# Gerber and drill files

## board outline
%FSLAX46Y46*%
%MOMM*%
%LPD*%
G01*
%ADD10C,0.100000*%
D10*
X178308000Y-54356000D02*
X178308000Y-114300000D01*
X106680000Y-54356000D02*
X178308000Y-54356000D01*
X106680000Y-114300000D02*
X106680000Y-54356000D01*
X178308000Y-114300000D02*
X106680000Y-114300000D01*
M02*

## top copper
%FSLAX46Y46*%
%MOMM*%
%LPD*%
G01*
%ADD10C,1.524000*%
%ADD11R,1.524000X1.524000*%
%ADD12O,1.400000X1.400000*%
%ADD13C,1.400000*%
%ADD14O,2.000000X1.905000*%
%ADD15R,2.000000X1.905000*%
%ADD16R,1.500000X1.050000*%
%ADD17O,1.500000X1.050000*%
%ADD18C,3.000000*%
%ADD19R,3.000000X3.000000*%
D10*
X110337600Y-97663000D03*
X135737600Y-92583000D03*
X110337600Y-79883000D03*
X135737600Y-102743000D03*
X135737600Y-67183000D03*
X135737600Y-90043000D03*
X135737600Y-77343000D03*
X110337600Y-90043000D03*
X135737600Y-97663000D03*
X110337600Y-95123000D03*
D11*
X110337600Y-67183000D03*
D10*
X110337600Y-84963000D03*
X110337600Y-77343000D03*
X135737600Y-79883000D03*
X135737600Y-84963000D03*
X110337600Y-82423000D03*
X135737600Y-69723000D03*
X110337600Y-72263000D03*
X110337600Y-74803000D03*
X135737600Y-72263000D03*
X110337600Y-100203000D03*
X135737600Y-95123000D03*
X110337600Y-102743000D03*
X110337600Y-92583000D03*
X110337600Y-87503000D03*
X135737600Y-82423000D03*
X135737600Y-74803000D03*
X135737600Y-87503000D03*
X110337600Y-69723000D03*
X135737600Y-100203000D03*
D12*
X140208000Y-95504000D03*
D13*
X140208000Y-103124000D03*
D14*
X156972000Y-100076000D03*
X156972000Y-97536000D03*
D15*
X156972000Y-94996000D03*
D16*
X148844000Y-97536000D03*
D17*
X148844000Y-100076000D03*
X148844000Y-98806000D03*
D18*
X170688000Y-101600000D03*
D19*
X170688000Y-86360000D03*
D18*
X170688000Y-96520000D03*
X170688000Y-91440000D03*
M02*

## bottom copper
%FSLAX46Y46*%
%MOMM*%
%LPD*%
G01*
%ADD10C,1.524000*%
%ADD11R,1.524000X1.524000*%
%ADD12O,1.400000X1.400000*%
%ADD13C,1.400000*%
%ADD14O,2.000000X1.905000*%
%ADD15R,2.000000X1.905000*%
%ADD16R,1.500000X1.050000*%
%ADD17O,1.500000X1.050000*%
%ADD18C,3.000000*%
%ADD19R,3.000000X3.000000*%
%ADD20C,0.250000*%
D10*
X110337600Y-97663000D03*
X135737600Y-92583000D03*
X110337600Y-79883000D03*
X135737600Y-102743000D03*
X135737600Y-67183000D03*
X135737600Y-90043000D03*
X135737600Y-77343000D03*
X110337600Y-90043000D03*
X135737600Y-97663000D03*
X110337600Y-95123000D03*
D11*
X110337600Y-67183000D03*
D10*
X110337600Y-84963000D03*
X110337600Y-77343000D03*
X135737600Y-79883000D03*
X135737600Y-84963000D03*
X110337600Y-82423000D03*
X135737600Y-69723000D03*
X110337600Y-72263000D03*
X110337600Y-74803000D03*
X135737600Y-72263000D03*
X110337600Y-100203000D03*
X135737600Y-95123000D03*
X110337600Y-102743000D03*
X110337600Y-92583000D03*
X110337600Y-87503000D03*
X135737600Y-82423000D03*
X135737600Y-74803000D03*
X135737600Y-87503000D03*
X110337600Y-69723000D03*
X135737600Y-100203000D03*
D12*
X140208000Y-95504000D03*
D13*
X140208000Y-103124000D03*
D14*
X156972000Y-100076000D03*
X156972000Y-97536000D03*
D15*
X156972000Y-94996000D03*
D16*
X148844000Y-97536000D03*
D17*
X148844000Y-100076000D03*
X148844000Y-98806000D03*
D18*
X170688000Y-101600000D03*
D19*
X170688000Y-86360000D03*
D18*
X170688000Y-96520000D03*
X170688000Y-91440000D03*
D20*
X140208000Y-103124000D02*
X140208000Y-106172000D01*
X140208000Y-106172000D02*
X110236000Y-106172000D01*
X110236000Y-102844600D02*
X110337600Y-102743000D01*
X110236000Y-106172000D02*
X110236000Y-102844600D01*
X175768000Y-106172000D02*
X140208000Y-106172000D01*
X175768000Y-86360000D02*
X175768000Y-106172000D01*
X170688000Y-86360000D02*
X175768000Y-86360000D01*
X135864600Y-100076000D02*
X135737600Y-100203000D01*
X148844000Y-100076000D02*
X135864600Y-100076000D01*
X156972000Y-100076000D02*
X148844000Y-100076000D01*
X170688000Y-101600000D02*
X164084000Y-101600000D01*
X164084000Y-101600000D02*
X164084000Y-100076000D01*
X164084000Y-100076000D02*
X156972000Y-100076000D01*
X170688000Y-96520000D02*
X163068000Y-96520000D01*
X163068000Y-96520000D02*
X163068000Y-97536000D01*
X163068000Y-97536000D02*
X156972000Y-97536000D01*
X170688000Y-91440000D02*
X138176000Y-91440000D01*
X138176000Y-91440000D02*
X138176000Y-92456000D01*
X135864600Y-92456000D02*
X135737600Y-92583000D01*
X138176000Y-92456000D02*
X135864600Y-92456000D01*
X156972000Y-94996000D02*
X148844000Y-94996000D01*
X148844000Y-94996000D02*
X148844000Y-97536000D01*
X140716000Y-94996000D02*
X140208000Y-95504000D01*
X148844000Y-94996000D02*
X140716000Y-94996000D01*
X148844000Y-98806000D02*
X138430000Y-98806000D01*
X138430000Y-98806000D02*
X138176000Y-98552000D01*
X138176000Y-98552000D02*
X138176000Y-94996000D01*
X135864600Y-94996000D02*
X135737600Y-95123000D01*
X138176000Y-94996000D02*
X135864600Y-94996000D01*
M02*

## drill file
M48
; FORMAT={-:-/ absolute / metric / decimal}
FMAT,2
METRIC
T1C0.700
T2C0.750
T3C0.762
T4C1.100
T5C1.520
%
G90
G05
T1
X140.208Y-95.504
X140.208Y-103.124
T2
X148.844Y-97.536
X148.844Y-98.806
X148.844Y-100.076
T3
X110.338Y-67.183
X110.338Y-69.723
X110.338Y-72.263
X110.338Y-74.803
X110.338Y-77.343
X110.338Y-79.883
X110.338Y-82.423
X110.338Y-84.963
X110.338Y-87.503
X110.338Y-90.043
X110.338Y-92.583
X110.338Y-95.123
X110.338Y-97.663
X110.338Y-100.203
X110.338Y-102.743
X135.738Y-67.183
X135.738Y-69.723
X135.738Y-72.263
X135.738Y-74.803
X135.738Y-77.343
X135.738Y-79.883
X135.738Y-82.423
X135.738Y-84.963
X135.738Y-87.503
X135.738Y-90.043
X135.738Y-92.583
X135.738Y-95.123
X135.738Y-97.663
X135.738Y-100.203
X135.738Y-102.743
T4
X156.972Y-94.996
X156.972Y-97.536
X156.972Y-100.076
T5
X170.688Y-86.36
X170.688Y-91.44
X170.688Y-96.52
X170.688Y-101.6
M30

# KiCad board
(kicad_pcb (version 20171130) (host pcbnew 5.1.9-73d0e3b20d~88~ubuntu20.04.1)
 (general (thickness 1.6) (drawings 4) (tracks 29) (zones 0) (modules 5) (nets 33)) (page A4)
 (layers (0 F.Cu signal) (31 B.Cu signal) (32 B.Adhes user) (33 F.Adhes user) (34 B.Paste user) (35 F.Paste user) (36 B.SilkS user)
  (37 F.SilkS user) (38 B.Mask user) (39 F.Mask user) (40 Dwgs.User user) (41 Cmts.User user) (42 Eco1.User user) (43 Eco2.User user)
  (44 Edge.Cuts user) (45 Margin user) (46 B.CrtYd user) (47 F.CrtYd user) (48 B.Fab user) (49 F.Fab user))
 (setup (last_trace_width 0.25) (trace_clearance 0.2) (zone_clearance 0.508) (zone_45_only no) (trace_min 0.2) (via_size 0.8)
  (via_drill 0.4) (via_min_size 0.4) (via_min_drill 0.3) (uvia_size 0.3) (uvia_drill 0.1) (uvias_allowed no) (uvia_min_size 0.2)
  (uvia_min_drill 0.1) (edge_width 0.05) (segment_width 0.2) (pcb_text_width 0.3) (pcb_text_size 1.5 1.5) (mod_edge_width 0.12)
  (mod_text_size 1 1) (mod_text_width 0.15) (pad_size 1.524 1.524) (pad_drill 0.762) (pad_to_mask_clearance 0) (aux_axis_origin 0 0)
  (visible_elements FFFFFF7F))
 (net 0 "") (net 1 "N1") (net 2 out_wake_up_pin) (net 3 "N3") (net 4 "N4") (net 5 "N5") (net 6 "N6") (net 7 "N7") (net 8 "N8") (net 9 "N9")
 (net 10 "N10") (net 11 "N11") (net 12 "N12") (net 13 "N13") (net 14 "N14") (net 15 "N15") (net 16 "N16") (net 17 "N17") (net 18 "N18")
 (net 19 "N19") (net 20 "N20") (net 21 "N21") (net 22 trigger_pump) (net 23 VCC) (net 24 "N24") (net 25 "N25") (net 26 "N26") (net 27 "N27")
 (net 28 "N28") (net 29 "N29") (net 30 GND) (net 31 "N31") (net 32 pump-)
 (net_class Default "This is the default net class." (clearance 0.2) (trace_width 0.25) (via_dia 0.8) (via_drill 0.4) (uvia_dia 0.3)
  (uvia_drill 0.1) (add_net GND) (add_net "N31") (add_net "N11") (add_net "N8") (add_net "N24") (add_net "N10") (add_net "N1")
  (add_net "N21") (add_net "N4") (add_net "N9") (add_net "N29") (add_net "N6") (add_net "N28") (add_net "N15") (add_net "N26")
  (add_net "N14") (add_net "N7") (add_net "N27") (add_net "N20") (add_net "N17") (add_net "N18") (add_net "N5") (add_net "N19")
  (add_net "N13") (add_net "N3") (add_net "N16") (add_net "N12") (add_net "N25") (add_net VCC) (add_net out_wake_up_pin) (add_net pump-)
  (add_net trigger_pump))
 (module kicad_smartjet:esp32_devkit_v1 (layer F.Cu) (at 121.92 58.42)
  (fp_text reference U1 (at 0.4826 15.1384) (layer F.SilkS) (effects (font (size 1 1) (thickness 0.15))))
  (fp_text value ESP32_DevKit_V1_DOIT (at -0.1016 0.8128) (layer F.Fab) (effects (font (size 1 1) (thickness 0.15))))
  (pad 13 thru_hole circle (at -11.5824 39.243) (size 1.524 1.524) (drill 0.762) (layers *.Cu *.Mask) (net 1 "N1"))
  (pad 20 thru_hole circle (at 13.8176 34.163) (size 1.524 1.524) (drill 0.762) (layers *.Cu *.Mask) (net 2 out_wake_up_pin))
  (pad 6 thru_hole circle (at -11.5824 21.463) (size 1.524 1.524) (drill 0.762) (layers *.Cu *.Mask) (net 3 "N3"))
  (pad 16 thru_hole circle (at 13.8176 44.323) (size 1.524 1.524) (drill 0.762) (layers *.Cu *.Mask) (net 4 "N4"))
  (pad 30 thru_hole circle (at 13.8176 8.763) (size 1.524 1.524) (drill 0.762) (layers *.Cu *.Mask) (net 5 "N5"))
  (pad 21 thru_hole circle (at 13.8176 31.623) (size 1.524 1.524) (drill 0.762) (layers *.Cu *.Mask) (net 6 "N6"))
  (pad 26 thru_hole circle (at 13.8176 18.923) (size 1.524 1.524) (drill 0.762) (layers *.Cu *.Mask) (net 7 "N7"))
  (pad 10 thru_hole circle (at -11.5824 31.623) (size 1.524 1.524) (drill 0.762) (layers *.Cu *.Mask) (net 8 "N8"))
  (pad 18 thru_hole circle (at 13.8176 39.243) (size 1.524 1.524) (drill 0.762) (layers *.Cu *.Mask) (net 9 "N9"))
  (pad 12 thru_hole circle (at -11.5824 36.703) (size 1.524 1.524) (drill 0.762) (layers *.Cu *.Mask) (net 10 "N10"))
  (pad 1 thru_hole rect (at -11.5824 8.763) (size 1.524 1.524) (drill 0.762) (layers *.Cu *.Mask) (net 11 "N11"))
  (pad 8 thru_hole circle (at -11.5824 26.543) (size 1.524 1.524) (drill 0.762) (layers *.Cu *.Mask) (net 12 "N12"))
  (pad 5 thru_hole circle (at -11.5824 18.923) (size 1.524 1.524) (drill 0.762) (layers *.Cu *.Mask) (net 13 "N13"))
  (pad 25 thru_hole circle (at 13.8176 21.463) (size 1.524 1.524) (drill 0.762) (layers *.Cu *.Mask) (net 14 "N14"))
  (pad 23 thru_hole circle (at 13.8176 26.543) (size 1.524 1.524) (drill 0.762) (layers *.Cu *.Mask) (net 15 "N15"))
  (pad 7 thru_hole circle (at -11.5824 24.003) (size 1.524 1.524) (drill 0.762) (layers *.Cu *.Mask) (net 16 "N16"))
  (pad 29 thru_hole circle (at 13.8176 11.303) (size 1.524 1.524) (drill 0.762) (layers *.Cu *.Mask) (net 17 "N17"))
  (pad 3 thru_hole circle (at -11.5824 13.843) (size 1.524 1.524) (drill 0.762) (layers *.Cu *.Mask) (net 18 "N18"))
  (pad 4 thru_hole circle (at -11.5824 16.383) (size 1.524 1.524) (drill 0.762) (layers *.Cu *.Mask) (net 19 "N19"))
  (pad 28 thru_hole circle (at 13.8176 13.843) (size 1.524 1.524) (drill 0.762) (layers *.Cu *.Mask) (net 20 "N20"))
  (pad 14 thru_hole circle (at -11.5824 41.783) (size 1.524 1.524) (drill 0.762) (layers *.Cu *.Mask) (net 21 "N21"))
  (pad 19 thru_hole circle (at 13.8176 36.703) (size 1.524 1.524) (drill 0.762) (layers *.Cu *.Mask) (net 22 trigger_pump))
  (pad 15 thru_hole circle (at -11.5824 44.323) (size 1.524 1.524) (drill 0.762) (layers *.Cu *.Mask) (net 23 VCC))
  (pad 11 thru_hole circle (at -11.5824 34.163) (size 1.524 1.524) (drill 0.762) (layers *.Cu *.Mask) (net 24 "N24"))
  (pad 9 thru_hole circle (at -11.5824 29.083) (size 1.524 1.524) (drill 0.762) (layers *.Cu *.Mask) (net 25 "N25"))
  (pad 24 thru_hole circle (at 13.8176 24.003) (size 1.524 1.524) (drill 0.762) (layers *.Cu *.Mask) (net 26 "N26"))
  (pad 27 thru_hole circle (at 13.8176 16.383) (size 1.524 1.524) (drill 0.762) (layers *.Cu *.Mask) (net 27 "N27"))
  (pad 22 thru_hole circle (at 13.8176 29.083) (size 1.524 1.524) (drill 0.762) (layers *.Cu *.Mask) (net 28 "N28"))
  (pad 2 thru_hole circle (at -11.5824 11.303) (size 1.524 1.524) (drill 0.762) (layers *.Cu *.Mask) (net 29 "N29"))
  (pad 17 thru_hole circle (at 13.8176 41.783) (size 1.524 1.524) (drill 0.762) (layers *.Cu *.Mask) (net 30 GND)))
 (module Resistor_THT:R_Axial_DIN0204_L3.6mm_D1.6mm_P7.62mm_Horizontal (layer F.Cu) (at 140.208 103.124 90)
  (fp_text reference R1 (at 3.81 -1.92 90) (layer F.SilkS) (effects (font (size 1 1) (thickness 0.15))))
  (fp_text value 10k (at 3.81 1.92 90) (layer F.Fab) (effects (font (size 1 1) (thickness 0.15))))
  (pad 2 thru_hole oval (at 7.62 0 90) (size 1.4 1.4) (drill 0.7) (layers *.Cu *.Mask) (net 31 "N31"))
  (pad 1 thru_hole circle (at 0 0 90) (size 1.4 1.4) (drill 0.7) (layers *.Cu *.Mask) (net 23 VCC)))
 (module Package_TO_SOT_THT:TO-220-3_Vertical (layer F.Cu) (at 156.972 94.996 270)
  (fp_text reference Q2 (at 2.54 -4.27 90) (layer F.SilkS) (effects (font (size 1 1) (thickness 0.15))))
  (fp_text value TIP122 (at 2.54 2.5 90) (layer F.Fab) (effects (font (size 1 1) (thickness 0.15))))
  (pad 3 thru_hole oval (at 5.08 0 270) (size 1.905 2) (drill 1.1) (layers *.Cu *.Mask) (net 30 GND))
  (pad 2 thru_hole oval (at 2.54 0 270) (size 1.905 2) (drill 1.1) (layers *.Cu *.Mask) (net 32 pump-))
  (pad 1 thru_hole rect (at 0 0 270) (size 1.905 2) (drill 1.1) (layers *.Cu *.Mask) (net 31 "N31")))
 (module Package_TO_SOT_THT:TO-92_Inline (layer F.Cu) (at 148.844 97.536 270)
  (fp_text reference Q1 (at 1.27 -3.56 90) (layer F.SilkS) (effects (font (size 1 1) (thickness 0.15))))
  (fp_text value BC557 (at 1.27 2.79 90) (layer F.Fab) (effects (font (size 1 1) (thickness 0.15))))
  (pad 1 thru_hole rect (at 0 0 270) (size 1.05 1.5) (drill 0.75) (layers *.Cu *.Mask) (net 31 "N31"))
  (pad 3 thru_hole oval (at 2.54 0 270) (size 1.05 1.5) (drill 0.75) (layers *.Cu *.Mask) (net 30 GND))
  (pad 2 thru_hole oval (at 1.27 0 270) (size 1.05 1.5) (drill 0.75) (layers *.Cu *.Mask) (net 22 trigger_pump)))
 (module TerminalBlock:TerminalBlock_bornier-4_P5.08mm (layer F.Cu) (at 170.688 86.36 270)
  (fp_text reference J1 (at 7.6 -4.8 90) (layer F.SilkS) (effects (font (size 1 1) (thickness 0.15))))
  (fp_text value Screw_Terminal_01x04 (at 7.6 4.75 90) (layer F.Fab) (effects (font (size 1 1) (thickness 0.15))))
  (pad 4 thru_hole circle (at 15.24 0 270) (size 3 3) (drill 1.52) (layers *.Cu *.Mask) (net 30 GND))
  (pad 1 thru_hole rect (at 0 0 270) (size 3 3) (drill 1.52) (layers *.Cu *.Mask) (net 23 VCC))
  (pad 3 thru_hole circle (at 10.16 0 270) (size 3 3) (drill 1.52) (layers *.Cu *.Mask) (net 32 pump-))
  (pad 2 thru_hole circle (at 5.08 0 270) (size 3 3) (drill 1.52) (layers *.Cu *.Mask) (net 2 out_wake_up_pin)))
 (gr_line (start 178.308 54.356) (end 178.308 114.3) (layer Edge.Cuts) (width 0.1))
 (gr_line (start 106.68 54.356) (end 178.308 54.356) (layer Edge.Cuts) (width 0.1))
 (gr_line (start 106.68 114.3) (end 106.68 54.356) (layer Edge.Cuts) (width 0.1))
 (gr_line (start 178.308 114.3) (end 106.68 114.3) (layer Edge.Cuts) (width 0.1))
 (segment (start 140.208 103.124) (end 140.208 106.172) (width 0.25) (layer B.Cu) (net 23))
 (segment (start 140.208 106.172) (end 110.236 106.172) (width 0.25) (layer B.Cu) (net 23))
 (segment (start 110.236 102.8446) (end 110.3376 102.743) (width 0.25) (layer B.Cu) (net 23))
 (segment (start 110.236 106.172) (end 110.236 102.8446) (width 0.25) (layer B.Cu) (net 23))
 (segment (start 175.768 106.172) (end 140.208 106.172) (width 0.25) (layer B.Cu) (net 23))
 (segment (start 175.768 86.36) (end 175.768 106.172) (width 0.25) (layer B.Cu) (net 23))
 (segment (start 170.688 86.36) (end 175.768 86.36) (width 0.25) (layer B.Cu) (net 23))
 (segment (start 135.8646 100.076) (end 135.7376 100.203) (width 0.25) (layer B.Cu) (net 30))
 (segment (start 148.844 100.076) (end 135.8646 100.076) (width 0.25) (layer B.Cu) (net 30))
 (segment (start 156.972 100.076) (end 148.844 100.076) (width 0.25) (layer B.Cu) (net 30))
 (segment (start 170.688 101.6) (end 164.084 101.6) (width 0.25) (layer B.Cu) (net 30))
 (segment (start 164.084 101.6) (end 164.084 100.076) (width 0.25) (layer B.Cu) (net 30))
 (segment (start 164.084 100.076) (end 156.972 100.076) (width 0.25) (layer B.Cu) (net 30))
 (segment (start 170.688 96.52) (end 163.068 96.52) (width 0.25) (layer B.Cu) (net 32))
 (segment (start 163.068 96.52) (end 163.068 97.536) (width 0.25) (layer B.Cu) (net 32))
 (segment (start 163.068 97.536) (end 156.972 97.536) (width 0.25) (layer B.Cu) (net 32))
 (segment (start 170.688 91.44) (end 138.176 91.44) (width 0.25) (layer B.Cu) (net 2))
 (segment (start 138.176 91.44) (end 138.176 92.456) (width 0.25) (layer B.Cu) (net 2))
 (segment (start 135.8646 92.456) (end 135.7376 92.583) (width 0.25) (layer B.Cu) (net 2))
 (segment (start 138.176 92.456) (end 135.8646 92.456) (width 0.25) (layer B.Cu) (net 2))
 (segment (start 156.972 94.996) (end 148.844 94.996) (width 0.25) (layer B.Cu) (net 31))
 (segment (start 148.844 94.996) (end 148.844 97.536) (width 0.25) (layer B.Cu) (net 31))
 (segment (start 140.716 94.996) (end 140.208 95.504) (width 0.25) (layer B.Cu) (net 31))
 (segment (start 148.844 94.996) (end 140.716 94.996) (width 0.25) (layer B.Cu) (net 31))
 (segment (start 148.844 98.806) (end 138.43 98.806) (width 0.25) (layer B.Cu) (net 22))
 (segment (start 138.43 98.806) (end 138.176 98.552) (width 0.25) (layer B.Cu) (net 22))
 (segment (start 138.176 98.552) (end 138.176 94.996) (width 0.25) (layer B.Cu) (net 22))
 (segment (start 135.8646 94.996) (end 135.7376 95.123) (width 0.25) (layer B.Cu) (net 22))
 (segment (start 138.176 94.996) (end 135.8646 94.996) (width 0.25) (layer B.Cu) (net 22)))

